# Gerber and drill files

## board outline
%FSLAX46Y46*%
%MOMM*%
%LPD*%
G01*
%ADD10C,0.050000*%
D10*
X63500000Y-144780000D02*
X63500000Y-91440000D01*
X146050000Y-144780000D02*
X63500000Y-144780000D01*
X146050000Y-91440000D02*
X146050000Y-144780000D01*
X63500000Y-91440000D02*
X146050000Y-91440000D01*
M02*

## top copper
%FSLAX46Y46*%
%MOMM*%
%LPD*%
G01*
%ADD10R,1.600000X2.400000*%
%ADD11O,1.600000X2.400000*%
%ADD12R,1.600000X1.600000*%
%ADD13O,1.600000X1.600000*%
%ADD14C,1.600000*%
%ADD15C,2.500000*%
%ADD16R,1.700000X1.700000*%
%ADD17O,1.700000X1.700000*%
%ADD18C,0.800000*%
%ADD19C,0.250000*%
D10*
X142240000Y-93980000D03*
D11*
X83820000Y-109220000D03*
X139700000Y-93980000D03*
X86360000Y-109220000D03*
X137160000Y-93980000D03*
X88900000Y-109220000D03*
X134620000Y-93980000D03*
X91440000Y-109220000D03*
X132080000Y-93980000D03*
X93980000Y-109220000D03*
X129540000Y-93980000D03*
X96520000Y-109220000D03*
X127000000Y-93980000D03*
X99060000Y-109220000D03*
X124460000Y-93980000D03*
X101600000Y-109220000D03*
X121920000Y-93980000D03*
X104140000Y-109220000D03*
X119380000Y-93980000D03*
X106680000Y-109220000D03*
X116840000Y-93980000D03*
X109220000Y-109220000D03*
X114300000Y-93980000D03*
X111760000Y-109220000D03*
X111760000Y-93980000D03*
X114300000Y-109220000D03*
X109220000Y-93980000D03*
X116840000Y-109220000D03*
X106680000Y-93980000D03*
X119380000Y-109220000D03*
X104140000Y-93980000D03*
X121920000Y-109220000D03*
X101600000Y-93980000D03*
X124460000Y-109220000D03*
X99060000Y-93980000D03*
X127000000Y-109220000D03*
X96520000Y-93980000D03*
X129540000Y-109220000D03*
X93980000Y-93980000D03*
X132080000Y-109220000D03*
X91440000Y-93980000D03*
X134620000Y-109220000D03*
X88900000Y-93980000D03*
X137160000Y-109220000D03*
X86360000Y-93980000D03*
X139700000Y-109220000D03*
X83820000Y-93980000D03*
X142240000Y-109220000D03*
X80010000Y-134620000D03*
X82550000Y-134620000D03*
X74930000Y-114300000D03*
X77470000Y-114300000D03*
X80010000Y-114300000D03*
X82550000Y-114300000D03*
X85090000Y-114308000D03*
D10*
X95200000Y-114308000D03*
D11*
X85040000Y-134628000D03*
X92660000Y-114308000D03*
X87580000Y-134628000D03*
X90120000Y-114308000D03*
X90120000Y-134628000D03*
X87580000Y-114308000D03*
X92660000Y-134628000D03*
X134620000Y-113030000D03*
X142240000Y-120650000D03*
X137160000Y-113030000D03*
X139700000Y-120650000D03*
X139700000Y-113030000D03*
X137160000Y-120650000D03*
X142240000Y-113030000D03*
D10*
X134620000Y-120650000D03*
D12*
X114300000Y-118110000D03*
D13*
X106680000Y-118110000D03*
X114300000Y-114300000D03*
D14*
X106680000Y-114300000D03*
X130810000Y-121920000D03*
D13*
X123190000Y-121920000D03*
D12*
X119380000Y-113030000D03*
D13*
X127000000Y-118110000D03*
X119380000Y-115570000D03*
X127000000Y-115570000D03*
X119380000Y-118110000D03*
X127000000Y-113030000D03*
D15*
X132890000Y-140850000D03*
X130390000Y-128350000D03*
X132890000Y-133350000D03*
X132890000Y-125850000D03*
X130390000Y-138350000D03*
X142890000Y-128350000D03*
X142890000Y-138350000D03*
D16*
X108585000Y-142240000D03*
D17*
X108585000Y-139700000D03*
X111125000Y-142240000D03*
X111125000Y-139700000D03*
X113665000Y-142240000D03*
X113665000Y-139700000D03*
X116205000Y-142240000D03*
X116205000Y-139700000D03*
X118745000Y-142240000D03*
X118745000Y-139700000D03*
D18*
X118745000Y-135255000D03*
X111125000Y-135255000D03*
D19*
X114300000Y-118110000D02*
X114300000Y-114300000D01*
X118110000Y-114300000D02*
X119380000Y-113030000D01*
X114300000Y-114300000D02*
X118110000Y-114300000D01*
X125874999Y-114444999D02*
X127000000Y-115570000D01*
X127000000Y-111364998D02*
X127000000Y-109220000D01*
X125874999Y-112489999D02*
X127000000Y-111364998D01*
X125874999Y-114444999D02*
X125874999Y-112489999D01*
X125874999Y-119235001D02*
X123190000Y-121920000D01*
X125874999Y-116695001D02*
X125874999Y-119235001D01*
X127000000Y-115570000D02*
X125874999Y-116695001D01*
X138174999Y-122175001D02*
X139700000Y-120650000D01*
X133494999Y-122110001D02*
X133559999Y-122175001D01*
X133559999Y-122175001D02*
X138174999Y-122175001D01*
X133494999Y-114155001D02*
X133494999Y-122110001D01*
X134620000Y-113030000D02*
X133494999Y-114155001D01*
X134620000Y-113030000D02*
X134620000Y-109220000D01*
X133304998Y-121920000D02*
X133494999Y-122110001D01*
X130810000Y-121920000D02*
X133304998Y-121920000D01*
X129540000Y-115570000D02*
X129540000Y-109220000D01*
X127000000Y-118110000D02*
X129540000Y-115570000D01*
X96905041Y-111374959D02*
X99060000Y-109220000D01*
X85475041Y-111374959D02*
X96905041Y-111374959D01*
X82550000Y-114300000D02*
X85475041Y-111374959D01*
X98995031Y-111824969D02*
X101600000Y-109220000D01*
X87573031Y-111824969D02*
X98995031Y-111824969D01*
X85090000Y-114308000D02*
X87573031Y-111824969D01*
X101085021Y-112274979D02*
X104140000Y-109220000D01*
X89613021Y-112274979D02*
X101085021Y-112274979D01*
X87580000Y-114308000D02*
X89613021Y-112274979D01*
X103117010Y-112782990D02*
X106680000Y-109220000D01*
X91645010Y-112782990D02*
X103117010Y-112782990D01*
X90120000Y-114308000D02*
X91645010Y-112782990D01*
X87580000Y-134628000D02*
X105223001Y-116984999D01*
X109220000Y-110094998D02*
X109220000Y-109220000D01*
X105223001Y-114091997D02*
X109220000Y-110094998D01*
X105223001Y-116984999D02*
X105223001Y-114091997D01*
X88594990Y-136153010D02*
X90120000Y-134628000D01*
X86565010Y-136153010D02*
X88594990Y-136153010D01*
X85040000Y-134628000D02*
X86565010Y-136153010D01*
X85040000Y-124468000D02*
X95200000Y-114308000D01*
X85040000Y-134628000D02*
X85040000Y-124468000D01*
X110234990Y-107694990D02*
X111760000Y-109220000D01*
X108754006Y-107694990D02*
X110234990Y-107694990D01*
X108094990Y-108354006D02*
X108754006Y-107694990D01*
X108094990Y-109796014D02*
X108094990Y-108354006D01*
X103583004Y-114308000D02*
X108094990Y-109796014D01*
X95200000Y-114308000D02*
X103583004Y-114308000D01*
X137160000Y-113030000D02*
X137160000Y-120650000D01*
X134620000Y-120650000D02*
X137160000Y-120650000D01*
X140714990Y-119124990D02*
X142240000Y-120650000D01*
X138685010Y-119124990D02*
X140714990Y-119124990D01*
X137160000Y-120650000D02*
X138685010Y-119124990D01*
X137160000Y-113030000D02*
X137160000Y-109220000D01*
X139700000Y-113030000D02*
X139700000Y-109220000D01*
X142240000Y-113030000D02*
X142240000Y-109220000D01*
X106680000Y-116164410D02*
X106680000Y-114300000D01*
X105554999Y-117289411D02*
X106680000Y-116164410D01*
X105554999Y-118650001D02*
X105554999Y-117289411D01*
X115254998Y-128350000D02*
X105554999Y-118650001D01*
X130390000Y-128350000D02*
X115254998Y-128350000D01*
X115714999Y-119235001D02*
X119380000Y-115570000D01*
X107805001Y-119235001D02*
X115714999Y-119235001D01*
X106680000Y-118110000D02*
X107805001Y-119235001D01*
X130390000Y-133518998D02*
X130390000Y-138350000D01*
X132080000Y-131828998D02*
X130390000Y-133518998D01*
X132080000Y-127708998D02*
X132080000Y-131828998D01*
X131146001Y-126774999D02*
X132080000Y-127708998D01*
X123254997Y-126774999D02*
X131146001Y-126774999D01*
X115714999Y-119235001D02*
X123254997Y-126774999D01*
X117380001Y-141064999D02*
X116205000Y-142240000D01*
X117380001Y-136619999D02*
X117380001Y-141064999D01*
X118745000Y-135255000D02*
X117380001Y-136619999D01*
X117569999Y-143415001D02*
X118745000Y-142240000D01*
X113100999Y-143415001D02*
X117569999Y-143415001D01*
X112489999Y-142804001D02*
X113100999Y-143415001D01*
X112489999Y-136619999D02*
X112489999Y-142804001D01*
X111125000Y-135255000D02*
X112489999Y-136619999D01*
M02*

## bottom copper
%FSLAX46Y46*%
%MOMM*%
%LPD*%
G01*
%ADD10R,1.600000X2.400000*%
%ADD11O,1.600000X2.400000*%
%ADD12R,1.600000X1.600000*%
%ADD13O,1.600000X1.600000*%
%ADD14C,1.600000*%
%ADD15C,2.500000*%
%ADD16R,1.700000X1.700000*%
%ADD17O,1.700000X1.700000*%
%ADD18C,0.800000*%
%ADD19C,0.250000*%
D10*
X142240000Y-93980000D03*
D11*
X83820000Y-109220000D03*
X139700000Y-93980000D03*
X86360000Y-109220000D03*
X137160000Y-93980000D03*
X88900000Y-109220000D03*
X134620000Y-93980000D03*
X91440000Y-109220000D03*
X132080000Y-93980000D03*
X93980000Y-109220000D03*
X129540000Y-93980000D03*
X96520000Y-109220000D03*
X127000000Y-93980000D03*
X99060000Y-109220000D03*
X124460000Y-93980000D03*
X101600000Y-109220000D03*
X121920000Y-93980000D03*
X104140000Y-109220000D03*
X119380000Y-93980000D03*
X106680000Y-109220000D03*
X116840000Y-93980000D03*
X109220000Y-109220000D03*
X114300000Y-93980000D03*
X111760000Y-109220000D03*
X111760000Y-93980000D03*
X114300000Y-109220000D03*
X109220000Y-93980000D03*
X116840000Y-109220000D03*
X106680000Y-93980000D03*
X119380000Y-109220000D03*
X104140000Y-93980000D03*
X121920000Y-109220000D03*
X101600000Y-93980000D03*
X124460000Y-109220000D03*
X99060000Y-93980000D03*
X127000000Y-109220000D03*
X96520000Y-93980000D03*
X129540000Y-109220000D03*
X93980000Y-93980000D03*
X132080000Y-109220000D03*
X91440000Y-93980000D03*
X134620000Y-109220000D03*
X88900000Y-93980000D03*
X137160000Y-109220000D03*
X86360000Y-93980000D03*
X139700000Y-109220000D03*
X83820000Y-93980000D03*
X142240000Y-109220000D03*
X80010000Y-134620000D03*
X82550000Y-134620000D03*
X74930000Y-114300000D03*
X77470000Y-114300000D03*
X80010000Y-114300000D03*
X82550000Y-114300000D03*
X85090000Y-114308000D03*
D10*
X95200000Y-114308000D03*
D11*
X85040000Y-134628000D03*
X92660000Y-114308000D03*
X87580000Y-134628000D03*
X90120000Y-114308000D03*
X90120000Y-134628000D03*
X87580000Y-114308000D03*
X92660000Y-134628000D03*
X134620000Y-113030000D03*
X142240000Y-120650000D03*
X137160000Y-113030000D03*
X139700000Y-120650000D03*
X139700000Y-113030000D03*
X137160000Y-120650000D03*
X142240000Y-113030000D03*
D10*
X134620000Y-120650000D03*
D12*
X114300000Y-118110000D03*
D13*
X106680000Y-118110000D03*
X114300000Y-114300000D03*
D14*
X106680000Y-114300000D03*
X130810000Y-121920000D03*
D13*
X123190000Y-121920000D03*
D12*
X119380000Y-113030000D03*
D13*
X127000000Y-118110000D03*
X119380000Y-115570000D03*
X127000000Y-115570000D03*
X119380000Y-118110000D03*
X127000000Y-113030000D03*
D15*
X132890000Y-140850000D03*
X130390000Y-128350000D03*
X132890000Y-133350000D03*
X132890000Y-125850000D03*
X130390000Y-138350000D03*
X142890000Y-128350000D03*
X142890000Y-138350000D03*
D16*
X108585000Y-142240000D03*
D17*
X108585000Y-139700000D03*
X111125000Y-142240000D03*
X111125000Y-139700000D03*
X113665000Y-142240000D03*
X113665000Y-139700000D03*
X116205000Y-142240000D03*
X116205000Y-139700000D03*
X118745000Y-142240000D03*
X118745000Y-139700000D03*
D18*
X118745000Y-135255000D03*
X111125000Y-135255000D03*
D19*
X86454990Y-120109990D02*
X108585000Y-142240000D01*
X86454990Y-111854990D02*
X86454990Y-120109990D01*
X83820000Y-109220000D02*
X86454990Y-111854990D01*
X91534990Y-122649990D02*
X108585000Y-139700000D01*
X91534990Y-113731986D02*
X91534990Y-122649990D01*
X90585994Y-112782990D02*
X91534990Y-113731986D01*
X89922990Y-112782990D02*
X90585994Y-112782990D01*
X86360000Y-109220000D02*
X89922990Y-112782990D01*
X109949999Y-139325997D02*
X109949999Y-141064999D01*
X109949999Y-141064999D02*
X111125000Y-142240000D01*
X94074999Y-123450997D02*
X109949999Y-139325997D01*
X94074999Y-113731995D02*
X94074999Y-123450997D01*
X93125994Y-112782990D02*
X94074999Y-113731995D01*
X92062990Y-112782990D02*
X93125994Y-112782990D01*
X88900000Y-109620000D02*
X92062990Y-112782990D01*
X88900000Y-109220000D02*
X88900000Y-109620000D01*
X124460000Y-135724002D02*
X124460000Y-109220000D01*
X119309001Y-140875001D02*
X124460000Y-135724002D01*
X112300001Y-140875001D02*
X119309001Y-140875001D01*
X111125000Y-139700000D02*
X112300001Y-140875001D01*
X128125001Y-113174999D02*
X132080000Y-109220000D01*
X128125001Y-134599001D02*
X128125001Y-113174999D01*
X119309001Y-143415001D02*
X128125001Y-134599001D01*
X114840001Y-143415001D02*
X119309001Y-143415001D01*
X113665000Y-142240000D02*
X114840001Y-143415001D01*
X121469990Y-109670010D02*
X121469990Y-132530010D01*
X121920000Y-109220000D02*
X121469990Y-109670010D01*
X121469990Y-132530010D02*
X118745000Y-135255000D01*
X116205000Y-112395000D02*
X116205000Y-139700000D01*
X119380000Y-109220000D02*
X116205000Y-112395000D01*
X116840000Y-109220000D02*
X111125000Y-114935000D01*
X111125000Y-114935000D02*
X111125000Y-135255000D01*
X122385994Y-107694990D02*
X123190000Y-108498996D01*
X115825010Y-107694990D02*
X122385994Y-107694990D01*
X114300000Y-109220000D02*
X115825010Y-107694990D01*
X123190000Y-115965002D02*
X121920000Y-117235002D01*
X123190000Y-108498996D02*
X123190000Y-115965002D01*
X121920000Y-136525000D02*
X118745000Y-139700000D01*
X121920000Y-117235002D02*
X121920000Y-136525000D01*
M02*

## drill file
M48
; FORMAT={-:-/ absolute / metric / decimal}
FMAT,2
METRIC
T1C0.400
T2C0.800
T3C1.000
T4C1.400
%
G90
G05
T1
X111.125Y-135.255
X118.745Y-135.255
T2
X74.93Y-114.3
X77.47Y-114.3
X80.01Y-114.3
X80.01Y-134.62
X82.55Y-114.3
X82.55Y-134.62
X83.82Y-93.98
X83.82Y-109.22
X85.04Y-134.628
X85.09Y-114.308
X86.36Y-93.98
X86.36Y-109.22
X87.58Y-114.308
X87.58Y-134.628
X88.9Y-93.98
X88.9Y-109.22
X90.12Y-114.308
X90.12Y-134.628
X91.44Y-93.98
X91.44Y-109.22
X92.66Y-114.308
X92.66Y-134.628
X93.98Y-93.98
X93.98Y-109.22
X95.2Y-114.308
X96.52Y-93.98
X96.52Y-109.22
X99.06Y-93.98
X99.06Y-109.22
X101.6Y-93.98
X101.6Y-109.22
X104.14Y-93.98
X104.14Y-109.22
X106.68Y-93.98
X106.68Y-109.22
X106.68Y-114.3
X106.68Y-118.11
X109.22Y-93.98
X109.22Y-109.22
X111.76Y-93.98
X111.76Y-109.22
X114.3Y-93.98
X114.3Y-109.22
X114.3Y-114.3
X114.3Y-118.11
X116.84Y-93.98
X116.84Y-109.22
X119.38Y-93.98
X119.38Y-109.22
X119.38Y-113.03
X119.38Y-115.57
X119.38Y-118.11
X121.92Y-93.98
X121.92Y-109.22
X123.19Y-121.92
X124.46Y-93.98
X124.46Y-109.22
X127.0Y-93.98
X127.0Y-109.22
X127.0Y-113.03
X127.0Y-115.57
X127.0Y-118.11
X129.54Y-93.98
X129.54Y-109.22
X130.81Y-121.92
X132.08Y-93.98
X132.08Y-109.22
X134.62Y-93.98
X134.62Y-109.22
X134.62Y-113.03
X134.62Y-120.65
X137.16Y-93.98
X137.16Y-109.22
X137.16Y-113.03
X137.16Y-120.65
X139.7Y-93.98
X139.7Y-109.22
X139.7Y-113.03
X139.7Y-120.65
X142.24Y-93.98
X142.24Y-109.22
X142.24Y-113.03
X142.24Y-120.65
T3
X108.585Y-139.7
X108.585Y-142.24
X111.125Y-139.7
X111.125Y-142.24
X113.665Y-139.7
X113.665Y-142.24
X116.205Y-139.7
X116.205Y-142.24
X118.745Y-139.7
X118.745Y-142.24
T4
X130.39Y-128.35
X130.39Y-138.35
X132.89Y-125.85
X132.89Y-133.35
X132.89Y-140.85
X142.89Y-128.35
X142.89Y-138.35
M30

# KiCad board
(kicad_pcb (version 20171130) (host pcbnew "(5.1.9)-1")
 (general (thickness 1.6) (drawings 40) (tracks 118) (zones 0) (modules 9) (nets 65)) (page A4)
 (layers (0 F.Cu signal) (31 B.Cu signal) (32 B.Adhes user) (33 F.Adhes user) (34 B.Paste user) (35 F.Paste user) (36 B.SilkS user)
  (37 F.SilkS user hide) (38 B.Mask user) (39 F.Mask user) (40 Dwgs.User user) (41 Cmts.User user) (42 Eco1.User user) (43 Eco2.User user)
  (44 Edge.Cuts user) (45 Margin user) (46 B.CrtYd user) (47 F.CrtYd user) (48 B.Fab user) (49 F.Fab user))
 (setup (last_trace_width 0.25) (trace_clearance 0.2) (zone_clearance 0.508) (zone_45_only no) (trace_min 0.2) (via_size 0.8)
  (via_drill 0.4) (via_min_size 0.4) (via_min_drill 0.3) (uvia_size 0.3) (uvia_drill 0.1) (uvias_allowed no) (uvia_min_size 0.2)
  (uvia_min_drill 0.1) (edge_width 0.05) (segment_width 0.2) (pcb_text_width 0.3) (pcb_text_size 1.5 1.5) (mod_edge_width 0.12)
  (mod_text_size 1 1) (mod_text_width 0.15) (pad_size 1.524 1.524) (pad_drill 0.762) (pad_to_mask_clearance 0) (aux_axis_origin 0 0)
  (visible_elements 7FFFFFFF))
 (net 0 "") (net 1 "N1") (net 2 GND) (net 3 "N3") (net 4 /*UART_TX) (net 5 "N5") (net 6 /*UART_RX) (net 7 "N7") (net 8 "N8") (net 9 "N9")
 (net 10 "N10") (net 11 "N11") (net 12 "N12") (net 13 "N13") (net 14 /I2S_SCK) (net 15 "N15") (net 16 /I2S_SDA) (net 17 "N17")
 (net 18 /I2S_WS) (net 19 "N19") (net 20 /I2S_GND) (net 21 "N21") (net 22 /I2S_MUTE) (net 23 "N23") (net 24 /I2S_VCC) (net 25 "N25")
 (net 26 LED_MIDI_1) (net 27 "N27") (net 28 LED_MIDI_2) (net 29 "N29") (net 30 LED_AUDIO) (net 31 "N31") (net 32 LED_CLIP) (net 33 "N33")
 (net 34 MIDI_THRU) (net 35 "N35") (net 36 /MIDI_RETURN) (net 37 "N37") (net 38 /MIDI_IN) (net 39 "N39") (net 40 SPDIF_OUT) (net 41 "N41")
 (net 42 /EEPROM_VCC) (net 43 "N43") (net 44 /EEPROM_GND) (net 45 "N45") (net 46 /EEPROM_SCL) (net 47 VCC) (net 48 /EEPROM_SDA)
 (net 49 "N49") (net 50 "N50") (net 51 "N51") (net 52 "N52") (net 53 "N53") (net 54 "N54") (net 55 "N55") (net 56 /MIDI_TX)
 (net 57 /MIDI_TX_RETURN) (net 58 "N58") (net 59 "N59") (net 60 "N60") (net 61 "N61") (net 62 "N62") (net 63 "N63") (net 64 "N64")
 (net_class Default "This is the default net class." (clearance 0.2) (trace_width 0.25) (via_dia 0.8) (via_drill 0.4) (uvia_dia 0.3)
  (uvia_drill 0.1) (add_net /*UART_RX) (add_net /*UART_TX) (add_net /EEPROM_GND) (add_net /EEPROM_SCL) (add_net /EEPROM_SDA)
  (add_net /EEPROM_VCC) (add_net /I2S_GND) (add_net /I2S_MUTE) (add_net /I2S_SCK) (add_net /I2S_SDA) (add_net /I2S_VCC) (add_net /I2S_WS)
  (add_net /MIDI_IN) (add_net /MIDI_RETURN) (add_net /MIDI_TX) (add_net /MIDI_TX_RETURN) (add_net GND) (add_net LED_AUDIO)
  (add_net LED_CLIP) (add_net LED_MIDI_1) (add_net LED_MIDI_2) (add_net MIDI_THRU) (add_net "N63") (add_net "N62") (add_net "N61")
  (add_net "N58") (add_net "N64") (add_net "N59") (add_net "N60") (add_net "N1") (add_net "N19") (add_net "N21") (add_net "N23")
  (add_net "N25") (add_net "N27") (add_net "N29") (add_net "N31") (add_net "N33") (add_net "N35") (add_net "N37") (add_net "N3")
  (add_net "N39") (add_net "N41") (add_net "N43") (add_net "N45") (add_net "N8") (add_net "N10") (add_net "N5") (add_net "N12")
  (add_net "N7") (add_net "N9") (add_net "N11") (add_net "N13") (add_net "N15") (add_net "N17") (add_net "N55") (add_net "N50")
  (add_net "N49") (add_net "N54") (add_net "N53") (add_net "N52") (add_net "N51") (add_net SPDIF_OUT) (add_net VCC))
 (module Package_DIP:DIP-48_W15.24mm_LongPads (layer F.Cu) (at 142.24 93.98 270)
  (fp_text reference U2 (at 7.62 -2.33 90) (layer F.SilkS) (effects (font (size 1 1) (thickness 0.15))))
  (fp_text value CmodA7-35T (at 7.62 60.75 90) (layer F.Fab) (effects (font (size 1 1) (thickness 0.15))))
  (pad 1 thru_hole rect (at 0 0 270) (size 2.4 1.6) (drill 0.8) (layers *.Cu *.Mask) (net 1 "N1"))
  (pad 25 thru_hole oval (at 15.24 58.42 270) (size 2.4 1.6) (drill 0.8) (layers *.Cu *.Mask) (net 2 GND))
  (pad 2 thru_hole oval (at 0 2.54 270) (size 2.4 1.6) (drill 0.8) (layers *.Cu *.Mask) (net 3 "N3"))
  (pad 26 thru_hole oval (at 15.24 55.88 270) (size 2.4 1.6) (drill 0.8) (layers *.Cu *.Mask) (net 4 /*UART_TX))
  (pad 3 thru_hole oval (at 0 5.08 270) (size 2.4 1.6) (drill 0.8) (layers *.Cu *.Mask) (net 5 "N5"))
  (pad 27 thru_hole oval (at 15.24 53.34 270) (size 2.4 1.6) (drill 0.8) (layers *.Cu *.Mask) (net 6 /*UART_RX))
  (pad 4 thru_hole oval (at 0 7.62 270) (size 2.4 1.6) (drill 0.8) (layers *.Cu *.Mask) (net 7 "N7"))
  (pad 28 thru_hole oval (at 15.24 50.8 270) (size 2.4 1.6) (drill 0.8) (layers *.Cu *.Mask) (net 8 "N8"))
  (pad 5 thru_hole oval (at 0 10.16 270) (size 2.4 1.6) (drill 0.8) (layers *.Cu *.Mask) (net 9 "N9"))
  (pad 29 thru_hole oval (at 15.24 48.26 270) (size 2.4 1.6) (drill 0.8) (layers *.Cu *.Mask) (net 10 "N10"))
  (pad 6 thru_hole oval (at 0 12.7 270) (size 2.4 1.6) (drill 0.8) (layers *.Cu *.Mask) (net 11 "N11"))
  (pad 30 thru_hole oval (at 15.24 45.72 270) (size 2.4 1.6) (drill 0.8) (layers *.Cu *.Mask) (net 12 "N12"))
  (pad 7 thru_hole oval (at 0 15.24 270) (size 2.4 1.6) (drill 0.8) (layers *.Cu *.Mask) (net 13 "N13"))
  (pad 31 thru_hole oval (at 15.24 43.18 270) (size 2.4 1.6) (drill 0.8) (layers *.Cu *.Mask) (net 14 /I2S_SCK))
  (pad 8 thru_hole oval (at 0 17.78 270) (size 2.4 1.6) (drill 0.8) (layers *.Cu *.Mask) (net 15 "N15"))
  (pad 32 thru_hole oval (at 15.24 40.64 270) (size 2.4 1.6) (drill 0.8) (layers *.Cu *.Mask) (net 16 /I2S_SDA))
  (pad 9 thru_hole oval (at 0 20.32 270) (size 2.4 1.6) (drill 0.8) (layers *.Cu *.Mask) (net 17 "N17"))
  (pad 33 thru_hole oval (at 15.24 38.1 270) (size 2.4 1.6) (drill 0.8) (layers *.Cu *.Mask) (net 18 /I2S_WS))
  (pad 10 thru_hole oval (at 0 22.86 270) (size 2.4 1.6) (drill 0.8) (layers *.Cu *.Mask) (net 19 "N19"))
  (pad 34 thru_hole oval (at 15.24 35.56 270) (size 2.4 1.6) (drill 0.8) (layers *.Cu *.Mask) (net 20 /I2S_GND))
  (pad 11 thru_hole oval (at 0 25.4 270) (size 2.4 1.6) (drill 0.8) (layers *.Cu *.Mask) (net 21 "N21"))
  (pad 35 thru_hole oval (at 15.24 33.02 270) (size 2.4 1.6) (drill 0.8) (layers *.Cu *.Mask) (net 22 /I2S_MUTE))
  (pad 12 thru_hole oval (at 0 27.94 270) (size 2.4 1.6) (drill 0.8) (layers *.Cu *.Mask) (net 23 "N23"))
  (pad 36 thru_hole oval (at 15.24 30.48 270) (size 2.4 1.6) (drill 0.8) (layers *.Cu *.Mask) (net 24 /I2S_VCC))
  (pad 13 thru_hole oval (at 0 30.48 270) (size 2.4 1.6) (drill 0.8) (layers *.Cu *.Mask) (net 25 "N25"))
  (pad 37 thru_hole oval (at 15.24 27.94 270) (size 2.4 1.6) (drill 0.8) (layers *.Cu *.Mask) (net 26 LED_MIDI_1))
  (pad 14 thru_hole oval (at 0 33.02 270) (size 2.4 1.6) (drill 0.8) (layers *.Cu *.Mask) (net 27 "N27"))
  (pad 38 thru_hole oval (at 15.24 25.4 270) (size 2.4 1.6) (drill 0.8) (layers *.Cu *.Mask) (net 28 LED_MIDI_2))
  (pad 15 thru_hole oval (at 0 35.56 270) (size 2.4 1.6) (drill 0.8) (layers *.Cu *.Mask) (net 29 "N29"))
  (pad 39 thru_hole oval (at 15.24 22.86 270) (size 2.4 1.6) (drill 0.8) (layers *.Cu *.Mask) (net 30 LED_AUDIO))
  (pad 16 thru_hole oval (at 0 38.1 270) (size 2.4 1.6) (drill 0.8) (layers *.Cu *.Mask) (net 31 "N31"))
  (pad 40 thru_hole oval (at 15.24 20.32 270) (size 2.4 1.6) (drill 0.8) (layers *.Cu *.Mask) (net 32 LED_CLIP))
  (pad 17 thru_hole oval (at 0 40.64 270) (size 2.4 1.6) (drill 0.8) (layers *.Cu *.Mask) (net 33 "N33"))
  (pad 41 thru_hole oval (at 15.24 17.78 270) (size 2.4 1.6) (drill 0.8) (layers *.Cu *.Mask) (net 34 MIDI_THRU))
  (pad 18 thru_hole oval (at 0 43.18 270) (size 2.4 1.6) (drill 0.8) (layers *.Cu *.Mask) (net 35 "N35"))
  (pad 42 thru_hole oval (at 15.24 15.24 270) (size 2.4 1.6) (drill 0.8) (layers *.Cu *.Mask) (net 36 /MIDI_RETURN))
  (pad 19 thru_hole oval (at 0 45.72 270) (size 2.4 1.6) (drill 0.8) (layers *.Cu *.Mask) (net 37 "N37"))
  (pad 43 thru_hole oval (at 15.24 12.7 270) (size 2.4 1.6) (drill 0.8) (layers *.Cu *.Mask) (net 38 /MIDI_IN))
  (pad 20 thru_hole oval (at 0 48.26 270) (size 2.4 1.6) (drill 0.8) (layers *.Cu *.Mask) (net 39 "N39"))
  (pad 44 thru_hole oval (at 15.24 10.16 270) (size 2.4 1.6) (drill 0.8) (layers *.Cu *.Mask) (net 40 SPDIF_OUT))
  (pad 21 thru_hole oval (at 0 50.8 270) (size 2.4 1.6) (drill 0.8) (layers *.Cu *.Mask) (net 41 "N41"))
  (pad 45 thru_hole oval (at 15.24 7.62 270) (size 2.4 1.6) (drill 0.8) (layers *.Cu *.Mask) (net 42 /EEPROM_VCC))
  (pad 22 thru_hole oval (at 0 53.34 270) (size 2.4 1.6) (drill 0.8) (layers *.Cu *.Mask) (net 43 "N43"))
  (pad 46 thru_hole oval (at 15.24 5.08 270) (size 2.4 1.6) (drill 0.8) (layers *.Cu *.Mask) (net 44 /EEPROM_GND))
  (pad 23 thru_hole oval (at 0 55.88 270) (size 2.4 1.6) (drill 0.8) (layers *.Cu *.Mask) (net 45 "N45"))
  (pad 47 thru_hole oval (at 15.24 2.54 270) (size 2.4 1.6) (drill 0.8) (layers *.Cu *.Mask) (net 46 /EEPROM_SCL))
  (pad 24 thru_hole oval (at 0 58.42 270) (size 2.4 1.6) (drill 0.8) (layers *.Cu *.Mask) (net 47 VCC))
  (pad 48 thru_hole oval (at 15.24 0 270) (size 2.4 1.6) (drill 0.8) (layers *.Cu *.Mask) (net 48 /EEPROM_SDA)))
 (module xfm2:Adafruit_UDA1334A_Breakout (layer F.Cu) (at 100.33 114.3 270)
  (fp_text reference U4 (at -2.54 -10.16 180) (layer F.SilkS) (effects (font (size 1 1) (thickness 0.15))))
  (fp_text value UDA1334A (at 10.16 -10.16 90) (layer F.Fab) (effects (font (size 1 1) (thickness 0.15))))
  (pad 15 thru_hole oval (at 20.32 20.32 270) (size 2.4 1.6) (drill 0.8) (layers *.Cu *.Mask) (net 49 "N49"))
  (pad 14 thru_hole oval (at 20.32 17.78 270) (size 2.4 1.6) (drill 0.8) (layers *.Cu *.Mask) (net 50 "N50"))
  (pad 9 thru_hole oval (at 0 25.4 270) (size 2.4 1.6) (drill 0.8) (layers *.Cu *.Mask) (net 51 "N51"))
  (pad 8 thru_hole oval (at 0 22.86 270) (size 2.4 1.6) (drill 0.8) (layers *.Cu *.Mask) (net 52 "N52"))
  (pad 7 thru_hole oval (at 0 20.32 270) (size 2.4 1.6) (drill 0.8) (layers *.Cu *.Mask) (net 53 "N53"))
  (pad 6 thru_hole oval (at 0 17.78 270) (size 2.4 1.6) (drill 0.8) (layers *.Cu *.Mask) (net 14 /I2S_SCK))
  (pad 5 thru_hole oval (at 0.008 15.24 270) (size 2.4 1.6) (drill 0.8) (layers *.Cu *.Mask) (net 16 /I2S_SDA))
  (pad 1 thru_hole rect (at 0.008 5.13 270) (size 2.4 1.6) (drill 0.8) (layers *.Cu *.Mask) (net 24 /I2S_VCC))
  (pad 13 thru_hole oval (at 20.328 15.29 270) (size 2.4 1.6) (drill 0.8) (layers *.Cu *.Mask) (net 24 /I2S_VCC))
  (pad 2 thru_hole oval (at 0.008 7.67 270) (size 2.4 1.6) (drill 0.8) (layers *.Cu *.Mask) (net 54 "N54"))
  (pad 12 thru_hole oval (at 20.328 12.75 270) (size 2.4 1.6) (drill 0.8) (layers *.Cu *.Mask) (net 22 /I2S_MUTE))
  (pad 3 thru_hole oval (at 0.008 10.21 270) (size 2.4 1.6) (drill 0.8) (layers *.Cu *.Mask) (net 20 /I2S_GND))
  (pad 11 thru_hole oval (at 20.328 10.21 270) (size 2.4 1.6) (drill 0.8) (layers *.Cu *.Mask) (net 24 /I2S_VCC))
  (pad 4 thru_hole oval (at 0.008 12.75 270) (size 2.4 1.6) (drill 0.8) (layers *.Cu *.Mask) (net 18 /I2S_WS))
  (pad 10 thru_hole oval (at 20.328 7.67 270) (size 2.4 1.6) (drill 0.8) (layers *.Cu *.Mask) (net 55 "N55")))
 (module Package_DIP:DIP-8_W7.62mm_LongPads (layer F.Cu) (at 134.62 120.65 90)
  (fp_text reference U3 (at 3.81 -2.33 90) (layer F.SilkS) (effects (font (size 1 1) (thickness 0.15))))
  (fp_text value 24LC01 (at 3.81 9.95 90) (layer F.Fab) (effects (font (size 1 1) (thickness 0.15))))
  (pad 8 thru_hole oval (at 7.62 0 90) (size 2.4 1.6) (drill 0.8) (layers *.Cu *.Mask) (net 42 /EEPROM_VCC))
  (pad 4 thru_hole oval (at 0 7.62 90) (size 2.4 1.6) (drill 0.8) (layers *.Cu *.Mask) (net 44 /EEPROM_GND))
  (pad 7 thru_hole oval (at 7.62 2.54 90) (size 2.4 1.6) (drill 0.8) (layers *.Cu *.Mask) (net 44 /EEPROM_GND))
  (pad 3 thru_hole oval (at 0 5.08 90) (size 2.4 1.6) (drill 0.8) (layers *.Cu *.Mask) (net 42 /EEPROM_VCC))
  (pad 6 thru_hole oval (at 7.62 5.08 90) (size 2.4 1.6) (drill 0.8) (layers *.Cu *.Mask) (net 46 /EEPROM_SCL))
  (pad 2 thru_hole oval (at 0 2.54 90) (size 2.4 1.6) (drill 0.8) (layers *.Cu *.Mask) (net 44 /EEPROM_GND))
  (pad 5 thru_hole oval (at 7.62 7.62 90) (size 2.4 1.6) (drill 0.8) (layers *.Cu *.Mask) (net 48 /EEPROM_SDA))
  (pad 1 thru_hole rect (at 0 0 90) (size 2.4 1.6) (drill 0.8) (layers *.Cu *.Mask) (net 44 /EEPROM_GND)))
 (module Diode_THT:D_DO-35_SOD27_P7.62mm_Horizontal (layer F.Cu) (at 114.3 118.11 180)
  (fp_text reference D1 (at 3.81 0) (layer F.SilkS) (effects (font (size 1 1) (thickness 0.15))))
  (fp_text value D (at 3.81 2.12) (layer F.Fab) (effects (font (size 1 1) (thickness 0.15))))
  (pad 1 thru_hole rect (at 0 0 180) (size 1.6 1.6) (drill 0.8) (layers *.Cu *.Mask) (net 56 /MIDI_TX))
  (pad 2 thru_hole oval (at 7.62 0 180) (size 1.6 1.6) (drill 0.8) (layers *.Cu *.Mask) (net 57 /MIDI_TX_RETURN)))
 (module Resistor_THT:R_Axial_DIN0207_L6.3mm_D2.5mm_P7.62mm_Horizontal (layer F.Cu) (at 106.68 114.3)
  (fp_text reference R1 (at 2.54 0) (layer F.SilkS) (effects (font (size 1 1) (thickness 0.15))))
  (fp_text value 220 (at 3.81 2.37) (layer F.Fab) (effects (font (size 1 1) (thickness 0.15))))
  (pad 2 thru_hole oval (at 7.62 0) (size 1.6 1.6) (drill 0.8) (layers *.Cu *.Mask) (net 56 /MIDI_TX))
  (pad 1 thru_hole circle (at 0 0) (size 1.6 1.6) (drill 0.8) (layers *.Cu *.Mask) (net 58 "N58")))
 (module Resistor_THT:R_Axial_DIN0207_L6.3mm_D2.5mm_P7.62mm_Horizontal (layer F.Cu) (at 130.81 121.92 180)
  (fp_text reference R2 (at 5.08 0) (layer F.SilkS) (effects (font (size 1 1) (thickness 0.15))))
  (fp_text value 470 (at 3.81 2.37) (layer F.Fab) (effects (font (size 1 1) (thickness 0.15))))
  (pad 1 thru_hole circle (at 0 0 180) (size 1.6 1.6) (drill 0.8) (layers *.Cu *.Mask) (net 42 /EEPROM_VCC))
  (pad 2 thru_hole oval (at 7.62 0 180) (size 1.6 1.6) (drill 0.8) (layers *.Cu *.Mask) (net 36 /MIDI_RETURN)))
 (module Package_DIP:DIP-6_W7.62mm (layer F.Cu) (at 119.38 113.03)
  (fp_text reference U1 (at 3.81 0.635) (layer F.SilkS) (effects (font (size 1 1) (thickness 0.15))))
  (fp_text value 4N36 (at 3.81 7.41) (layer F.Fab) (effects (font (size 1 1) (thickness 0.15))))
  (pad 1 thru_hole rect (at 0 0) (size 1.6 1.6) (drill 0.8) (layers *.Cu *.Mask) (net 56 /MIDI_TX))
  (pad 4 thru_hole oval (at 7.62 5.08) (size 1.6 1.6) (drill 0.8) (layers *.Cu *.Mask) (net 38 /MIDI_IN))
  (pad 2 thru_hole oval (at 0 2.54) (size 1.6 1.6) (drill 0.8) (layers *.Cu *.Mask) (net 57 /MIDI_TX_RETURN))
  (pad 5 thru_hole oval (at 7.62 2.54) (size 1.6 1.6) (drill 0.8) (layers *.Cu *.Mask) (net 36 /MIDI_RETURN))
  (pad 3 thru_hole oval (at 0 5.08) (size 1.6 1.6) (drill 0.8) (layers *.Cu *.Mask) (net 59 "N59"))
  (pad 6 thru_hole oval (at 7.62 0) (size 1.6 1.6) (drill 0.8) (layers *.Cu *.Mask) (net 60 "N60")))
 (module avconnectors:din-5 (layer F.Cu) (at 135.89 133.35 90)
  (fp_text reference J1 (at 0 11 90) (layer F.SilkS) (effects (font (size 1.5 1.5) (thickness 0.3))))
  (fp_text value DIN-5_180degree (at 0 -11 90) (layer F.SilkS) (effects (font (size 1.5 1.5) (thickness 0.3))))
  (pad 3 thru_hole circle (at -7.5 -3 90) (size 2.5 2.5) (drill 1.4) (layers *.Cu *.Mask) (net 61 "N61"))
  (pad 4 thru_hole circle (at 5 -5.5 90) (size 2.5 2.5) (drill 1.4) (layers *.Cu *.Mask) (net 58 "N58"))
  (pad 2 thru_hole circle (at 0 -3 90) (size 2.5 2.5) (drill 1.4) (layers *.Cu *.Mask) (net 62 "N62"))
  (pad 1 thru_hole circle (at 7.5 -3 90) (size 2.5 2.5) (drill 1.4) (layers *.Cu *.Mask) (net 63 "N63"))
  (pad 5 thru_hole circle (at -5 -5.5 90) (size 2.5 2.5) (drill 1.4) (layers *.Cu *.Mask) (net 57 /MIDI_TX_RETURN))
  (pad 6 thru_hole circle (at 5 7 90) (size 2.5 2.5) (drill 1.4) (layers *.Cu *.Mask))
  (pad 6 thru_hole circle (at -5 7 90) (size 2.5 2.5) (drill 1.4) (layers *.Cu *.Mask)))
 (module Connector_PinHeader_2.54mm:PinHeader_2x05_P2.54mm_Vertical (layer F.Cu) (at 108.585 142.24 90)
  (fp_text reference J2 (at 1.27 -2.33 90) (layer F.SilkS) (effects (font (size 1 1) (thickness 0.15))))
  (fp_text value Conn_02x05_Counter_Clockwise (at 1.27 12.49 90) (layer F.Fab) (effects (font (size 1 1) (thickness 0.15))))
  (pad 1 thru_hole rect (at 0 0 90) (size 1.7 1.7) (drill 1) (layers *.Cu *.Mask) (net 2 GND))
  (pad 2 thru_hole oval (at 2.54 0 90) (size 1.7 1.7) (drill 1) (layers *.Cu *.Mask) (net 4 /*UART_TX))
  (pad 3 thru_hole oval (at 0 2.54 90) (size 1.7 1.7) (drill 1) (layers *.Cu *.Mask) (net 6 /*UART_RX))
  (pad 4 thru_hole oval (at 2.54 2.54 90) (size 1.7 1.7) (drill 1) (layers *.Cu *.Mask) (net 34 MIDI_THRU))
  (pad 5 thru_hole oval (at 0 5.08 90) (size 1.7 1.7) (drill 1) (layers *.Cu *.Mask) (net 40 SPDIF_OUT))
  (pad 6 thru_hole oval (at 2.54 5.08 90) (size 1.7 1.7) (drill 1) (layers *.Cu *.Mask) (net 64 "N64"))
  (pad 7 thru_hole oval (at 0 7.62 90) (size 1.7 1.7) (drill 1) (layers *.Cu *.Mask) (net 32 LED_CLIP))
  (pad 8 thru_hole oval (at 2.54 7.62 90) (size 1.7 1.7) (drill 1) (layers *.Cu *.Mask) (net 30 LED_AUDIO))
  (pad 9 thru_hole oval (at 0 10.16 90) (size 1.7 1.7) (drill 1) (layers *.Cu *.Mask) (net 28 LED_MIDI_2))
  (pad 10 thru_hole oval (at 2.54 10.16 90) (size 1.7 1.7) (drill 1) (layers *.Cu *.Mask) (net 26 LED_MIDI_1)))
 (gr_line (start 63.5 144.78) (end 63.5 91.44) (layer Edge.Cuts) (width 0.05))
 (gr_line (start 146.05 144.78) (end 63.5 144.78) (layer Edge.Cuts) (width 0.05))
 (gr_line (start 146.05 91.44) (end 146.05 144.78) (layer Edge.Cuts) (width 0.05))
 (gr_line (start 63.5 91.44) (end 146.05 91.44) (layer Edge.Cuts) (width 0.05))
 (segment (start 86.45499 120.10999) (end 108.585 142.24) (width 0.25) (layer B.Cu) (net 2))
 (segment (start 86.45499 111.85499) (end 86.45499 120.10999) (width 0.25) (layer B.Cu) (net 2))
 (segment (start 83.82 109.22) (end 86.45499 111.85499) (width 0.25) (layer B.Cu) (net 2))
 (segment (start 114.3 118.11) (end 114.3 114.3) (width 0.25) (layer F.Cu) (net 56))
 (segment (start 118.11 114.3) (end 119.38 113.03) (width 0.25) (layer F.Cu) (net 56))
 (segment (start 114.3 114.3) (end 118.11 114.3) (width 0.25) (layer F.Cu) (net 56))
 (segment (start 125.874999 114.444999) (end 127 115.57) (width 0.25) (layer F.Cu) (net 36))
 (segment (start 127 111.364998) (end 127 109.22) (width 0.25) (layer F.Cu) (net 36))
 (segment (start 125.874999 112.489999) (end 127 111.364998) (width 0.25) (layer F.Cu) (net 36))
 (segment (start 125.874999 114.444999) (end 125.874999 112.489999) (width 0.25) (layer F.Cu) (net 36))
 (segment (start 125.874999 119.235001) (end 123.19 121.92) (width 0.25) (layer F.Cu) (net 36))
 (segment (start 125.874999 116.695001) (end 125.874999 119.235001) (width 0.25) (layer F.Cu) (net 36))
 (segment (start 127 115.57) (end 125.874999 116.695001) (width 0.25) (layer F.Cu) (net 36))
 (segment (start 138.174999 122.175001) (end 139.7 120.65) (width 0.25) (layer F.Cu) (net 42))
 (segment (start 133.494999 122.110001) (end 133.559999 122.175001) (width 0.25) (layer F.Cu) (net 42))
 (segment (start 133.559999 122.175001) (end 138.174999 122.175001) (width 0.25) (layer F.Cu) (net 42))
 (segment (start 133.494999 114.155001) (end 133.494999 122.110001) (width 0.25) (layer F.Cu) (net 42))
 (segment (start 134.62 113.03) (end 133.494999 114.155001) (width 0.25) (layer F.Cu) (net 42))
 (segment (start 134.62 113.03) (end 134.62 109.22) (width 0.25) (layer F.Cu) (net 42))
 (segment (start 133.304998 121.92) (end 133.494999 122.110001) (width 0.25) (layer F.Cu) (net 42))
 (segment (start 130.81 121.92) (end 133.304998 121.92) (width 0.25) (layer F.Cu) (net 42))
 (segment (start 129.54 115.57) (end 129.54 109.22) (width 0.25) (layer F.Cu) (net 38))
 (segment (start 127 118.11) (end 129.54 115.57) (width 0.25) (layer F.Cu) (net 38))
 (segment (start 96.905041 111.374959) (end 99.06 109.22) (width 0.25) (layer F.Cu) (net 14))
 (segment (start 85.475041 111.374959) (end 96.905041 111.374959) (width 0.25) (layer F.Cu) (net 14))
 (segment (start 82.55 114.3) (end 85.475041 111.374959) (width 0.25) (layer F.Cu) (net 14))
 (segment (start 98.995031 111.824969) (end 101.6 109.22) (width 0.25) (layer F.Cu) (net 16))
 (segment (start 87.573031 111.824969) (end 98.995031 111.824969) (width 0.25) (layer F.Cu) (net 16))
 (segment (start 85.09 114.308) (end 87.573031 111.824969) (width 0.25) (layer F.Cu) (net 16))
 (segment (start 101.085021 112.274979) (end 104.14 109.22) (width 0.25) (layer F.Cu) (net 18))
 (segment (start 89.613021 112.274979) (end 101.085021 112.274979) (width 0.25) (layer F.Cu) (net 18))
 (segment (start 87.58 114.308) (end 89.613021 112.274979) (width 0.25) (layer F.Cu) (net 18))
 (segment (start 103.11701 112.78299) (end 106.68 109.22) (width 0.25) (layer F.Cu) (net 20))
 (segment (start 91.64501 112.78299) (end 103.11701 112.78299) (width 0.25) (layer F.Cu) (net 20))
 (segment (start 90.12 114.308) (end 91.64501 112.78299) (width 0.25) (layer F.Cu) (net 20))
 (segment (start 87.58 134.628) (end 105.223001 116.984999) (width 0.25) (layer F.Cu) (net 22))
 (segment (start 109.22 110.094998) (end 109.22 109.22) (width 0.25) (layer F.Cu) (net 22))
 (segment (start 105.223001 114.091997) (end 109.22 110.094998) (width 0.25) (layer F.Cu) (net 22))
 (segment (start 105.223001 116.984999) (end 105.223001 114.091997) (width 0.25) (layer F.Cu) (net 22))
 (segment (start 88.59499 136.15301) (end 90.12 134.628) (width 0.25) (layer F.Cu) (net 24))
 (segment (start 86.56501 136.15301) (end 88.59499 136.15301) (width 0.25) (layer F.Cu) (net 24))
 (segment (start 85.04 134.628) (end 86.56501 136.15301) (width 0.25) (layer F.Cu) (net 24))
 (segment (start 85.04 124.468) (end 95.2 114.308) (width 0.25) (layer F.Cu) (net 24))
 (segment (start 85.04 134.628) (end 85.04 124.468) (width 0.25) (layer F.Cu) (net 24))
 (segment (start 110.23499 107.69499) (end 111.76 109.22) (width 0.25) (layer F.Cu) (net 24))
 (segment (start 108.754006 107.69499) (end 110.23499 107.69499) (width 0.25) (layer F.Cu) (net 24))
 (segment (start 108.09499 108.354006) (end 108.754006 107.69499) (width 0.25) (layer F.Cu) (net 24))
 (segment (start 108.09499 109.796014) (end 108.09499 108.354006) (width 0.25) (layer F.Cu) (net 24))
 (segment (start 103.583004 114.308) (end 108.09499 109.796014) (width 0.25) (layer F.Cu) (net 24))
 (segment (start 95.2 114.308) (end 103.583004 114.308) (width 0.25) (layer F.Cu) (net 24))
 (segment (start 137.16 113.03) (end 137.16 120.65) (width 0.25) (layer F.Cu) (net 44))
 (segment (start 134.62 120.65) (end 137.16 120.65) (width 0.25) (layer F.Cu) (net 44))
 (segment (start 140.71499 119.12499) (end 142.24 120.65) (width 0.25) (layer F.Cu) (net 44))
 (segment (start 138.68501 119.12499) (end 140.71499 119.12499) (width 0.25) (layer F.Cu) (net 44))
 (segment (start 137.16 120.65) (end 138.68501 119.12499) (width 0.25) (layer F.Cu) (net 44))
 (segment (start 137.16 113.03) (end 137.16 109.22) (width 0.25) (layer F.Cu) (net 44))
 (segment (start 139.7 113.03) (end 139.7 109.22) (width 0.25) (layer F.Cu) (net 46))
 (segment (start 142.24 113.03) (end 142.24 109.22) (width 0.25) (layer F.Cu) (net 48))
 (segment (start 106.68 116.16441) (end 106.68 114.3) (width 0.25) (layer F.Cu) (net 58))
 (segment (start 105.554999 117.289411) (end 106.68 116.16441) (width 0.25) (layer F.Cu) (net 58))
 (segment (start 105.554999 118.650001) (end 105.554999 117.289411) (width 0.25) (layer F.Cu) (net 58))
 (segment (start 115.254998 128.35) (end 105.554999 118.650001) (width 0.25) (layer F.Cu) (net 58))
 (segment (start 130.39 128.35) (end 115.254998 128.35) (width 0.25) (layer F.Cu) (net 58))
 (segment (start 115.714999 119.235001) (end 119.38 115.57) (width 0.25) (layer F.Cu) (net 57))
 (segment (start 107.805001 119.235001) (end 115.714999 119.235001) (width 0.25) (layer F.Cu) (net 57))
 (segment (start 106.68 118.11) (end 107.805001 119.235001) (width 0.25) (layer F.Cu) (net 57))
 (segment (start 130.39 133.518998) (end 130.39 138.35) (width 0.25) (layer F.Cu) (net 57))
 (segment (start 132.08 131.828998) (end 130.39 133.518998) (width 0.25) (layer F.Cu) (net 57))
 (segment (start 132.08 127.708998) (end 132.08 131.828998) (width 0.25) (layer F.Cu) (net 57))
 (segment (start 131.146001 126.774999) (end 132.08 127.708998) (width 0.25) (layer F.Cu) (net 57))
 (segment (start 123.254997 126.774999) (end 131.146001 126.774999) (width 0.25) (layer F.Cu) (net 57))
 (segment (start 115.714999 119.235001) (end 123.254997 126.774999) (width 0.25) (layer F.Cu) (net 57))
 (segment (start 91.53499 122.64999) (end 108.585 139.7) (width 0.25) (layer B.Cu) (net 4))
 (segment (start 91.53499 113.731986) (end 91.53499 122.64999) (width 0.25) (layer B.Cu) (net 4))
 (segment (start 90.585994 112.78299) (end 91.53499 113.731986) (width 0.25) (layer B.Cu) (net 4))
 (segment (start 89.92299 112.78299) (end 90.585994 112.78299) (width 0.25) (layer B.Cu) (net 4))
 (segment (start 86.36 109.22) (end 89.92299 112.78299) (width 0.25) (layer B.Cu) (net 4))
 (segment (start 109.949999 139.325997) (end 109.949999 141.064999) (width 0.25) (layer B.Cu) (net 6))
 (segment (start 109.949999 141.064999) (end 111.125 142.24) (width 0.25) (layer B.Cu) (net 6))
 (segment (start 94.074999 123.450997) (end 109.949999 139.325997) (width 0.25) (layer B.Cu) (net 6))
 (segment (start 94.074999 113.731995) (end 94.074999 123.450997) (width 0.25) (layer B.Cu) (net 6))
 (segment (start 93.125994 112.78299) (end 94.074999 113.731995) (width 0.25) (layer B.Cu) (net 6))
 (segment (start 92.06299 112.78299) (end 93.125994 112.78299) (width 0.25) (layer B.Cu) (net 6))
 (segment (start 88.9 109.62) (end 92.06299 112.78299) (width 0.25) (layer B.Cu) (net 6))
 (segment (start 88.9 109.22) (end 88.9 109.62) (width 0.25) (layer B.Cu) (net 6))
 (segment (start 124.46 135.724002) (end 124.46 109.22) (width 0.25) (layer B.Cu) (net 34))
 (segment (start 119.309001 140.875001) (end 124.46 135.724002) (width 0.25) (layer B.Cu) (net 34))
 (segment (start 112.300001 140.875001) (end 119.309001 140.875001) (width 0.25) (layer B.Cu) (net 34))
 (segment (start 111.125 139.7) (end 112.300001 140.875001) (width 0.25) (layer B.Cu) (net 34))
 (segment (start 128.125001 113.174999) (end 132.08 109.22) (width 0.25) (layer B.Cu) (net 40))
 (segment (start 128.125001 134.599001) (end 128.125001 113.174999) (width 0.25) (layer B.Cu) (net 40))
 (segment (start 119.309001 143.415001) (end 128.125001 134.599001) (width 0.25) (layer B.Cu) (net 40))
 (segment (start 114.840001 143.415001) (end 119.309001 143.415001) (width 0.25) (layer B.Cu) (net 40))
 (segment (start 113.665 142.24) (end 114.840001 143.415001) (width 0.25) (layer B.Cu) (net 40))
 (segment (start 121.46999 109.67001) (end 121.46999 132.53001) (width 0.25) (layer B.Cu) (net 32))
 (segment (start 121.92 109.22) (end 121.46999 109.67001) (width 0.25) (layer B.Cu) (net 32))
 (via (at 118.745 135.255) (size 0.8) (drill 0.4) (layers F.Cu B.Cu) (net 32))
 (segment (start 121.46999 132.53001) (end 118.745 135.255) (width 0.25) (layer B.Cu) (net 32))
 (segment (start 117.380001 141.064999) (end 116.205 142.24) (width 0.25) (layer F.Cu) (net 32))
 (segment (start 117.380001 136.619999) (end 117.380001 141.064999) (width 0.25) (layer F.Cu) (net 32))
 (segment (start 118.745 135.255) (end 117.380001 136.619999) (width 0.25) (layer F.Cu) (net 32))
 (segment (start 116.205 112.395) (end 116.205 139.7) (width 0.25) (layer B.Cu) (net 30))
 (segment (start 119.38 109.22) (end 116.205 112.395) (width 0.25) (layer B.Cu) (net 30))
 (segment (start 116.84 109.22) (end 111.125 114.935) (width 0.25) (layer B.Cu) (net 28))
 (via (at 111.125 135.255) (size 0.8) (drill 0.4) (layers F.Cu B.Cu) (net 28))
 (segment (start 111.125 114.935) (end 111.125 135.255) (width 0.25) (layer B.Cu) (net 28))
 (segment (start 117.569999 143.415001) (end 118.745 142.24) (width 0.25) (layer F.Cu) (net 28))
 (segment (start 113.100999 143.415001) (end 117.569999 143.415001) (width 0.25) (layer F.Cu) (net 28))
 (segment (start 112.489999 142.804001) (end 113.100999 143.415001) (width 0.25) (layer F.Cu) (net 28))
 (segment (start 112.489999 136.619999) (end 112.489999 142.804001) (width 0.25) (layer F.Cu) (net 28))
 (segment (start 111.125 135.255) (end 112.489999 136.619999) (width 0.25) (layer F.Cu) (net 28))
 (segment (start 122.385994 107.69499) (end 123.19 108.498996) (width 0.25) (layer B.Cu) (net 26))
 (segment (start 115.82501 107.69499) (end 122.385994 107.69499) (width 0.25) (layer B.Cu) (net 26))
 (segment (start 114.3 109.22) (end 115.82501 107.69499) (width 0.25) (layer B.Cu) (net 26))
 (segment (start 123.19 115.965002) (end 121.92 117.235002) (width 0.25) (layer B.Cu) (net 26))
 (segment (start 123.19 108.498996) (end 123.19 115.965002) (width 0.25) (layer B.Cu) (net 26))
 (segment (start 121.92 136.525) (end 118.745 139.7) (width 0.25) (layer B.Cu) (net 26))
 (segment (start 121.92 117.235002) (end 121.92 136.525) (width 0.25) (layer B.Cu) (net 26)))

